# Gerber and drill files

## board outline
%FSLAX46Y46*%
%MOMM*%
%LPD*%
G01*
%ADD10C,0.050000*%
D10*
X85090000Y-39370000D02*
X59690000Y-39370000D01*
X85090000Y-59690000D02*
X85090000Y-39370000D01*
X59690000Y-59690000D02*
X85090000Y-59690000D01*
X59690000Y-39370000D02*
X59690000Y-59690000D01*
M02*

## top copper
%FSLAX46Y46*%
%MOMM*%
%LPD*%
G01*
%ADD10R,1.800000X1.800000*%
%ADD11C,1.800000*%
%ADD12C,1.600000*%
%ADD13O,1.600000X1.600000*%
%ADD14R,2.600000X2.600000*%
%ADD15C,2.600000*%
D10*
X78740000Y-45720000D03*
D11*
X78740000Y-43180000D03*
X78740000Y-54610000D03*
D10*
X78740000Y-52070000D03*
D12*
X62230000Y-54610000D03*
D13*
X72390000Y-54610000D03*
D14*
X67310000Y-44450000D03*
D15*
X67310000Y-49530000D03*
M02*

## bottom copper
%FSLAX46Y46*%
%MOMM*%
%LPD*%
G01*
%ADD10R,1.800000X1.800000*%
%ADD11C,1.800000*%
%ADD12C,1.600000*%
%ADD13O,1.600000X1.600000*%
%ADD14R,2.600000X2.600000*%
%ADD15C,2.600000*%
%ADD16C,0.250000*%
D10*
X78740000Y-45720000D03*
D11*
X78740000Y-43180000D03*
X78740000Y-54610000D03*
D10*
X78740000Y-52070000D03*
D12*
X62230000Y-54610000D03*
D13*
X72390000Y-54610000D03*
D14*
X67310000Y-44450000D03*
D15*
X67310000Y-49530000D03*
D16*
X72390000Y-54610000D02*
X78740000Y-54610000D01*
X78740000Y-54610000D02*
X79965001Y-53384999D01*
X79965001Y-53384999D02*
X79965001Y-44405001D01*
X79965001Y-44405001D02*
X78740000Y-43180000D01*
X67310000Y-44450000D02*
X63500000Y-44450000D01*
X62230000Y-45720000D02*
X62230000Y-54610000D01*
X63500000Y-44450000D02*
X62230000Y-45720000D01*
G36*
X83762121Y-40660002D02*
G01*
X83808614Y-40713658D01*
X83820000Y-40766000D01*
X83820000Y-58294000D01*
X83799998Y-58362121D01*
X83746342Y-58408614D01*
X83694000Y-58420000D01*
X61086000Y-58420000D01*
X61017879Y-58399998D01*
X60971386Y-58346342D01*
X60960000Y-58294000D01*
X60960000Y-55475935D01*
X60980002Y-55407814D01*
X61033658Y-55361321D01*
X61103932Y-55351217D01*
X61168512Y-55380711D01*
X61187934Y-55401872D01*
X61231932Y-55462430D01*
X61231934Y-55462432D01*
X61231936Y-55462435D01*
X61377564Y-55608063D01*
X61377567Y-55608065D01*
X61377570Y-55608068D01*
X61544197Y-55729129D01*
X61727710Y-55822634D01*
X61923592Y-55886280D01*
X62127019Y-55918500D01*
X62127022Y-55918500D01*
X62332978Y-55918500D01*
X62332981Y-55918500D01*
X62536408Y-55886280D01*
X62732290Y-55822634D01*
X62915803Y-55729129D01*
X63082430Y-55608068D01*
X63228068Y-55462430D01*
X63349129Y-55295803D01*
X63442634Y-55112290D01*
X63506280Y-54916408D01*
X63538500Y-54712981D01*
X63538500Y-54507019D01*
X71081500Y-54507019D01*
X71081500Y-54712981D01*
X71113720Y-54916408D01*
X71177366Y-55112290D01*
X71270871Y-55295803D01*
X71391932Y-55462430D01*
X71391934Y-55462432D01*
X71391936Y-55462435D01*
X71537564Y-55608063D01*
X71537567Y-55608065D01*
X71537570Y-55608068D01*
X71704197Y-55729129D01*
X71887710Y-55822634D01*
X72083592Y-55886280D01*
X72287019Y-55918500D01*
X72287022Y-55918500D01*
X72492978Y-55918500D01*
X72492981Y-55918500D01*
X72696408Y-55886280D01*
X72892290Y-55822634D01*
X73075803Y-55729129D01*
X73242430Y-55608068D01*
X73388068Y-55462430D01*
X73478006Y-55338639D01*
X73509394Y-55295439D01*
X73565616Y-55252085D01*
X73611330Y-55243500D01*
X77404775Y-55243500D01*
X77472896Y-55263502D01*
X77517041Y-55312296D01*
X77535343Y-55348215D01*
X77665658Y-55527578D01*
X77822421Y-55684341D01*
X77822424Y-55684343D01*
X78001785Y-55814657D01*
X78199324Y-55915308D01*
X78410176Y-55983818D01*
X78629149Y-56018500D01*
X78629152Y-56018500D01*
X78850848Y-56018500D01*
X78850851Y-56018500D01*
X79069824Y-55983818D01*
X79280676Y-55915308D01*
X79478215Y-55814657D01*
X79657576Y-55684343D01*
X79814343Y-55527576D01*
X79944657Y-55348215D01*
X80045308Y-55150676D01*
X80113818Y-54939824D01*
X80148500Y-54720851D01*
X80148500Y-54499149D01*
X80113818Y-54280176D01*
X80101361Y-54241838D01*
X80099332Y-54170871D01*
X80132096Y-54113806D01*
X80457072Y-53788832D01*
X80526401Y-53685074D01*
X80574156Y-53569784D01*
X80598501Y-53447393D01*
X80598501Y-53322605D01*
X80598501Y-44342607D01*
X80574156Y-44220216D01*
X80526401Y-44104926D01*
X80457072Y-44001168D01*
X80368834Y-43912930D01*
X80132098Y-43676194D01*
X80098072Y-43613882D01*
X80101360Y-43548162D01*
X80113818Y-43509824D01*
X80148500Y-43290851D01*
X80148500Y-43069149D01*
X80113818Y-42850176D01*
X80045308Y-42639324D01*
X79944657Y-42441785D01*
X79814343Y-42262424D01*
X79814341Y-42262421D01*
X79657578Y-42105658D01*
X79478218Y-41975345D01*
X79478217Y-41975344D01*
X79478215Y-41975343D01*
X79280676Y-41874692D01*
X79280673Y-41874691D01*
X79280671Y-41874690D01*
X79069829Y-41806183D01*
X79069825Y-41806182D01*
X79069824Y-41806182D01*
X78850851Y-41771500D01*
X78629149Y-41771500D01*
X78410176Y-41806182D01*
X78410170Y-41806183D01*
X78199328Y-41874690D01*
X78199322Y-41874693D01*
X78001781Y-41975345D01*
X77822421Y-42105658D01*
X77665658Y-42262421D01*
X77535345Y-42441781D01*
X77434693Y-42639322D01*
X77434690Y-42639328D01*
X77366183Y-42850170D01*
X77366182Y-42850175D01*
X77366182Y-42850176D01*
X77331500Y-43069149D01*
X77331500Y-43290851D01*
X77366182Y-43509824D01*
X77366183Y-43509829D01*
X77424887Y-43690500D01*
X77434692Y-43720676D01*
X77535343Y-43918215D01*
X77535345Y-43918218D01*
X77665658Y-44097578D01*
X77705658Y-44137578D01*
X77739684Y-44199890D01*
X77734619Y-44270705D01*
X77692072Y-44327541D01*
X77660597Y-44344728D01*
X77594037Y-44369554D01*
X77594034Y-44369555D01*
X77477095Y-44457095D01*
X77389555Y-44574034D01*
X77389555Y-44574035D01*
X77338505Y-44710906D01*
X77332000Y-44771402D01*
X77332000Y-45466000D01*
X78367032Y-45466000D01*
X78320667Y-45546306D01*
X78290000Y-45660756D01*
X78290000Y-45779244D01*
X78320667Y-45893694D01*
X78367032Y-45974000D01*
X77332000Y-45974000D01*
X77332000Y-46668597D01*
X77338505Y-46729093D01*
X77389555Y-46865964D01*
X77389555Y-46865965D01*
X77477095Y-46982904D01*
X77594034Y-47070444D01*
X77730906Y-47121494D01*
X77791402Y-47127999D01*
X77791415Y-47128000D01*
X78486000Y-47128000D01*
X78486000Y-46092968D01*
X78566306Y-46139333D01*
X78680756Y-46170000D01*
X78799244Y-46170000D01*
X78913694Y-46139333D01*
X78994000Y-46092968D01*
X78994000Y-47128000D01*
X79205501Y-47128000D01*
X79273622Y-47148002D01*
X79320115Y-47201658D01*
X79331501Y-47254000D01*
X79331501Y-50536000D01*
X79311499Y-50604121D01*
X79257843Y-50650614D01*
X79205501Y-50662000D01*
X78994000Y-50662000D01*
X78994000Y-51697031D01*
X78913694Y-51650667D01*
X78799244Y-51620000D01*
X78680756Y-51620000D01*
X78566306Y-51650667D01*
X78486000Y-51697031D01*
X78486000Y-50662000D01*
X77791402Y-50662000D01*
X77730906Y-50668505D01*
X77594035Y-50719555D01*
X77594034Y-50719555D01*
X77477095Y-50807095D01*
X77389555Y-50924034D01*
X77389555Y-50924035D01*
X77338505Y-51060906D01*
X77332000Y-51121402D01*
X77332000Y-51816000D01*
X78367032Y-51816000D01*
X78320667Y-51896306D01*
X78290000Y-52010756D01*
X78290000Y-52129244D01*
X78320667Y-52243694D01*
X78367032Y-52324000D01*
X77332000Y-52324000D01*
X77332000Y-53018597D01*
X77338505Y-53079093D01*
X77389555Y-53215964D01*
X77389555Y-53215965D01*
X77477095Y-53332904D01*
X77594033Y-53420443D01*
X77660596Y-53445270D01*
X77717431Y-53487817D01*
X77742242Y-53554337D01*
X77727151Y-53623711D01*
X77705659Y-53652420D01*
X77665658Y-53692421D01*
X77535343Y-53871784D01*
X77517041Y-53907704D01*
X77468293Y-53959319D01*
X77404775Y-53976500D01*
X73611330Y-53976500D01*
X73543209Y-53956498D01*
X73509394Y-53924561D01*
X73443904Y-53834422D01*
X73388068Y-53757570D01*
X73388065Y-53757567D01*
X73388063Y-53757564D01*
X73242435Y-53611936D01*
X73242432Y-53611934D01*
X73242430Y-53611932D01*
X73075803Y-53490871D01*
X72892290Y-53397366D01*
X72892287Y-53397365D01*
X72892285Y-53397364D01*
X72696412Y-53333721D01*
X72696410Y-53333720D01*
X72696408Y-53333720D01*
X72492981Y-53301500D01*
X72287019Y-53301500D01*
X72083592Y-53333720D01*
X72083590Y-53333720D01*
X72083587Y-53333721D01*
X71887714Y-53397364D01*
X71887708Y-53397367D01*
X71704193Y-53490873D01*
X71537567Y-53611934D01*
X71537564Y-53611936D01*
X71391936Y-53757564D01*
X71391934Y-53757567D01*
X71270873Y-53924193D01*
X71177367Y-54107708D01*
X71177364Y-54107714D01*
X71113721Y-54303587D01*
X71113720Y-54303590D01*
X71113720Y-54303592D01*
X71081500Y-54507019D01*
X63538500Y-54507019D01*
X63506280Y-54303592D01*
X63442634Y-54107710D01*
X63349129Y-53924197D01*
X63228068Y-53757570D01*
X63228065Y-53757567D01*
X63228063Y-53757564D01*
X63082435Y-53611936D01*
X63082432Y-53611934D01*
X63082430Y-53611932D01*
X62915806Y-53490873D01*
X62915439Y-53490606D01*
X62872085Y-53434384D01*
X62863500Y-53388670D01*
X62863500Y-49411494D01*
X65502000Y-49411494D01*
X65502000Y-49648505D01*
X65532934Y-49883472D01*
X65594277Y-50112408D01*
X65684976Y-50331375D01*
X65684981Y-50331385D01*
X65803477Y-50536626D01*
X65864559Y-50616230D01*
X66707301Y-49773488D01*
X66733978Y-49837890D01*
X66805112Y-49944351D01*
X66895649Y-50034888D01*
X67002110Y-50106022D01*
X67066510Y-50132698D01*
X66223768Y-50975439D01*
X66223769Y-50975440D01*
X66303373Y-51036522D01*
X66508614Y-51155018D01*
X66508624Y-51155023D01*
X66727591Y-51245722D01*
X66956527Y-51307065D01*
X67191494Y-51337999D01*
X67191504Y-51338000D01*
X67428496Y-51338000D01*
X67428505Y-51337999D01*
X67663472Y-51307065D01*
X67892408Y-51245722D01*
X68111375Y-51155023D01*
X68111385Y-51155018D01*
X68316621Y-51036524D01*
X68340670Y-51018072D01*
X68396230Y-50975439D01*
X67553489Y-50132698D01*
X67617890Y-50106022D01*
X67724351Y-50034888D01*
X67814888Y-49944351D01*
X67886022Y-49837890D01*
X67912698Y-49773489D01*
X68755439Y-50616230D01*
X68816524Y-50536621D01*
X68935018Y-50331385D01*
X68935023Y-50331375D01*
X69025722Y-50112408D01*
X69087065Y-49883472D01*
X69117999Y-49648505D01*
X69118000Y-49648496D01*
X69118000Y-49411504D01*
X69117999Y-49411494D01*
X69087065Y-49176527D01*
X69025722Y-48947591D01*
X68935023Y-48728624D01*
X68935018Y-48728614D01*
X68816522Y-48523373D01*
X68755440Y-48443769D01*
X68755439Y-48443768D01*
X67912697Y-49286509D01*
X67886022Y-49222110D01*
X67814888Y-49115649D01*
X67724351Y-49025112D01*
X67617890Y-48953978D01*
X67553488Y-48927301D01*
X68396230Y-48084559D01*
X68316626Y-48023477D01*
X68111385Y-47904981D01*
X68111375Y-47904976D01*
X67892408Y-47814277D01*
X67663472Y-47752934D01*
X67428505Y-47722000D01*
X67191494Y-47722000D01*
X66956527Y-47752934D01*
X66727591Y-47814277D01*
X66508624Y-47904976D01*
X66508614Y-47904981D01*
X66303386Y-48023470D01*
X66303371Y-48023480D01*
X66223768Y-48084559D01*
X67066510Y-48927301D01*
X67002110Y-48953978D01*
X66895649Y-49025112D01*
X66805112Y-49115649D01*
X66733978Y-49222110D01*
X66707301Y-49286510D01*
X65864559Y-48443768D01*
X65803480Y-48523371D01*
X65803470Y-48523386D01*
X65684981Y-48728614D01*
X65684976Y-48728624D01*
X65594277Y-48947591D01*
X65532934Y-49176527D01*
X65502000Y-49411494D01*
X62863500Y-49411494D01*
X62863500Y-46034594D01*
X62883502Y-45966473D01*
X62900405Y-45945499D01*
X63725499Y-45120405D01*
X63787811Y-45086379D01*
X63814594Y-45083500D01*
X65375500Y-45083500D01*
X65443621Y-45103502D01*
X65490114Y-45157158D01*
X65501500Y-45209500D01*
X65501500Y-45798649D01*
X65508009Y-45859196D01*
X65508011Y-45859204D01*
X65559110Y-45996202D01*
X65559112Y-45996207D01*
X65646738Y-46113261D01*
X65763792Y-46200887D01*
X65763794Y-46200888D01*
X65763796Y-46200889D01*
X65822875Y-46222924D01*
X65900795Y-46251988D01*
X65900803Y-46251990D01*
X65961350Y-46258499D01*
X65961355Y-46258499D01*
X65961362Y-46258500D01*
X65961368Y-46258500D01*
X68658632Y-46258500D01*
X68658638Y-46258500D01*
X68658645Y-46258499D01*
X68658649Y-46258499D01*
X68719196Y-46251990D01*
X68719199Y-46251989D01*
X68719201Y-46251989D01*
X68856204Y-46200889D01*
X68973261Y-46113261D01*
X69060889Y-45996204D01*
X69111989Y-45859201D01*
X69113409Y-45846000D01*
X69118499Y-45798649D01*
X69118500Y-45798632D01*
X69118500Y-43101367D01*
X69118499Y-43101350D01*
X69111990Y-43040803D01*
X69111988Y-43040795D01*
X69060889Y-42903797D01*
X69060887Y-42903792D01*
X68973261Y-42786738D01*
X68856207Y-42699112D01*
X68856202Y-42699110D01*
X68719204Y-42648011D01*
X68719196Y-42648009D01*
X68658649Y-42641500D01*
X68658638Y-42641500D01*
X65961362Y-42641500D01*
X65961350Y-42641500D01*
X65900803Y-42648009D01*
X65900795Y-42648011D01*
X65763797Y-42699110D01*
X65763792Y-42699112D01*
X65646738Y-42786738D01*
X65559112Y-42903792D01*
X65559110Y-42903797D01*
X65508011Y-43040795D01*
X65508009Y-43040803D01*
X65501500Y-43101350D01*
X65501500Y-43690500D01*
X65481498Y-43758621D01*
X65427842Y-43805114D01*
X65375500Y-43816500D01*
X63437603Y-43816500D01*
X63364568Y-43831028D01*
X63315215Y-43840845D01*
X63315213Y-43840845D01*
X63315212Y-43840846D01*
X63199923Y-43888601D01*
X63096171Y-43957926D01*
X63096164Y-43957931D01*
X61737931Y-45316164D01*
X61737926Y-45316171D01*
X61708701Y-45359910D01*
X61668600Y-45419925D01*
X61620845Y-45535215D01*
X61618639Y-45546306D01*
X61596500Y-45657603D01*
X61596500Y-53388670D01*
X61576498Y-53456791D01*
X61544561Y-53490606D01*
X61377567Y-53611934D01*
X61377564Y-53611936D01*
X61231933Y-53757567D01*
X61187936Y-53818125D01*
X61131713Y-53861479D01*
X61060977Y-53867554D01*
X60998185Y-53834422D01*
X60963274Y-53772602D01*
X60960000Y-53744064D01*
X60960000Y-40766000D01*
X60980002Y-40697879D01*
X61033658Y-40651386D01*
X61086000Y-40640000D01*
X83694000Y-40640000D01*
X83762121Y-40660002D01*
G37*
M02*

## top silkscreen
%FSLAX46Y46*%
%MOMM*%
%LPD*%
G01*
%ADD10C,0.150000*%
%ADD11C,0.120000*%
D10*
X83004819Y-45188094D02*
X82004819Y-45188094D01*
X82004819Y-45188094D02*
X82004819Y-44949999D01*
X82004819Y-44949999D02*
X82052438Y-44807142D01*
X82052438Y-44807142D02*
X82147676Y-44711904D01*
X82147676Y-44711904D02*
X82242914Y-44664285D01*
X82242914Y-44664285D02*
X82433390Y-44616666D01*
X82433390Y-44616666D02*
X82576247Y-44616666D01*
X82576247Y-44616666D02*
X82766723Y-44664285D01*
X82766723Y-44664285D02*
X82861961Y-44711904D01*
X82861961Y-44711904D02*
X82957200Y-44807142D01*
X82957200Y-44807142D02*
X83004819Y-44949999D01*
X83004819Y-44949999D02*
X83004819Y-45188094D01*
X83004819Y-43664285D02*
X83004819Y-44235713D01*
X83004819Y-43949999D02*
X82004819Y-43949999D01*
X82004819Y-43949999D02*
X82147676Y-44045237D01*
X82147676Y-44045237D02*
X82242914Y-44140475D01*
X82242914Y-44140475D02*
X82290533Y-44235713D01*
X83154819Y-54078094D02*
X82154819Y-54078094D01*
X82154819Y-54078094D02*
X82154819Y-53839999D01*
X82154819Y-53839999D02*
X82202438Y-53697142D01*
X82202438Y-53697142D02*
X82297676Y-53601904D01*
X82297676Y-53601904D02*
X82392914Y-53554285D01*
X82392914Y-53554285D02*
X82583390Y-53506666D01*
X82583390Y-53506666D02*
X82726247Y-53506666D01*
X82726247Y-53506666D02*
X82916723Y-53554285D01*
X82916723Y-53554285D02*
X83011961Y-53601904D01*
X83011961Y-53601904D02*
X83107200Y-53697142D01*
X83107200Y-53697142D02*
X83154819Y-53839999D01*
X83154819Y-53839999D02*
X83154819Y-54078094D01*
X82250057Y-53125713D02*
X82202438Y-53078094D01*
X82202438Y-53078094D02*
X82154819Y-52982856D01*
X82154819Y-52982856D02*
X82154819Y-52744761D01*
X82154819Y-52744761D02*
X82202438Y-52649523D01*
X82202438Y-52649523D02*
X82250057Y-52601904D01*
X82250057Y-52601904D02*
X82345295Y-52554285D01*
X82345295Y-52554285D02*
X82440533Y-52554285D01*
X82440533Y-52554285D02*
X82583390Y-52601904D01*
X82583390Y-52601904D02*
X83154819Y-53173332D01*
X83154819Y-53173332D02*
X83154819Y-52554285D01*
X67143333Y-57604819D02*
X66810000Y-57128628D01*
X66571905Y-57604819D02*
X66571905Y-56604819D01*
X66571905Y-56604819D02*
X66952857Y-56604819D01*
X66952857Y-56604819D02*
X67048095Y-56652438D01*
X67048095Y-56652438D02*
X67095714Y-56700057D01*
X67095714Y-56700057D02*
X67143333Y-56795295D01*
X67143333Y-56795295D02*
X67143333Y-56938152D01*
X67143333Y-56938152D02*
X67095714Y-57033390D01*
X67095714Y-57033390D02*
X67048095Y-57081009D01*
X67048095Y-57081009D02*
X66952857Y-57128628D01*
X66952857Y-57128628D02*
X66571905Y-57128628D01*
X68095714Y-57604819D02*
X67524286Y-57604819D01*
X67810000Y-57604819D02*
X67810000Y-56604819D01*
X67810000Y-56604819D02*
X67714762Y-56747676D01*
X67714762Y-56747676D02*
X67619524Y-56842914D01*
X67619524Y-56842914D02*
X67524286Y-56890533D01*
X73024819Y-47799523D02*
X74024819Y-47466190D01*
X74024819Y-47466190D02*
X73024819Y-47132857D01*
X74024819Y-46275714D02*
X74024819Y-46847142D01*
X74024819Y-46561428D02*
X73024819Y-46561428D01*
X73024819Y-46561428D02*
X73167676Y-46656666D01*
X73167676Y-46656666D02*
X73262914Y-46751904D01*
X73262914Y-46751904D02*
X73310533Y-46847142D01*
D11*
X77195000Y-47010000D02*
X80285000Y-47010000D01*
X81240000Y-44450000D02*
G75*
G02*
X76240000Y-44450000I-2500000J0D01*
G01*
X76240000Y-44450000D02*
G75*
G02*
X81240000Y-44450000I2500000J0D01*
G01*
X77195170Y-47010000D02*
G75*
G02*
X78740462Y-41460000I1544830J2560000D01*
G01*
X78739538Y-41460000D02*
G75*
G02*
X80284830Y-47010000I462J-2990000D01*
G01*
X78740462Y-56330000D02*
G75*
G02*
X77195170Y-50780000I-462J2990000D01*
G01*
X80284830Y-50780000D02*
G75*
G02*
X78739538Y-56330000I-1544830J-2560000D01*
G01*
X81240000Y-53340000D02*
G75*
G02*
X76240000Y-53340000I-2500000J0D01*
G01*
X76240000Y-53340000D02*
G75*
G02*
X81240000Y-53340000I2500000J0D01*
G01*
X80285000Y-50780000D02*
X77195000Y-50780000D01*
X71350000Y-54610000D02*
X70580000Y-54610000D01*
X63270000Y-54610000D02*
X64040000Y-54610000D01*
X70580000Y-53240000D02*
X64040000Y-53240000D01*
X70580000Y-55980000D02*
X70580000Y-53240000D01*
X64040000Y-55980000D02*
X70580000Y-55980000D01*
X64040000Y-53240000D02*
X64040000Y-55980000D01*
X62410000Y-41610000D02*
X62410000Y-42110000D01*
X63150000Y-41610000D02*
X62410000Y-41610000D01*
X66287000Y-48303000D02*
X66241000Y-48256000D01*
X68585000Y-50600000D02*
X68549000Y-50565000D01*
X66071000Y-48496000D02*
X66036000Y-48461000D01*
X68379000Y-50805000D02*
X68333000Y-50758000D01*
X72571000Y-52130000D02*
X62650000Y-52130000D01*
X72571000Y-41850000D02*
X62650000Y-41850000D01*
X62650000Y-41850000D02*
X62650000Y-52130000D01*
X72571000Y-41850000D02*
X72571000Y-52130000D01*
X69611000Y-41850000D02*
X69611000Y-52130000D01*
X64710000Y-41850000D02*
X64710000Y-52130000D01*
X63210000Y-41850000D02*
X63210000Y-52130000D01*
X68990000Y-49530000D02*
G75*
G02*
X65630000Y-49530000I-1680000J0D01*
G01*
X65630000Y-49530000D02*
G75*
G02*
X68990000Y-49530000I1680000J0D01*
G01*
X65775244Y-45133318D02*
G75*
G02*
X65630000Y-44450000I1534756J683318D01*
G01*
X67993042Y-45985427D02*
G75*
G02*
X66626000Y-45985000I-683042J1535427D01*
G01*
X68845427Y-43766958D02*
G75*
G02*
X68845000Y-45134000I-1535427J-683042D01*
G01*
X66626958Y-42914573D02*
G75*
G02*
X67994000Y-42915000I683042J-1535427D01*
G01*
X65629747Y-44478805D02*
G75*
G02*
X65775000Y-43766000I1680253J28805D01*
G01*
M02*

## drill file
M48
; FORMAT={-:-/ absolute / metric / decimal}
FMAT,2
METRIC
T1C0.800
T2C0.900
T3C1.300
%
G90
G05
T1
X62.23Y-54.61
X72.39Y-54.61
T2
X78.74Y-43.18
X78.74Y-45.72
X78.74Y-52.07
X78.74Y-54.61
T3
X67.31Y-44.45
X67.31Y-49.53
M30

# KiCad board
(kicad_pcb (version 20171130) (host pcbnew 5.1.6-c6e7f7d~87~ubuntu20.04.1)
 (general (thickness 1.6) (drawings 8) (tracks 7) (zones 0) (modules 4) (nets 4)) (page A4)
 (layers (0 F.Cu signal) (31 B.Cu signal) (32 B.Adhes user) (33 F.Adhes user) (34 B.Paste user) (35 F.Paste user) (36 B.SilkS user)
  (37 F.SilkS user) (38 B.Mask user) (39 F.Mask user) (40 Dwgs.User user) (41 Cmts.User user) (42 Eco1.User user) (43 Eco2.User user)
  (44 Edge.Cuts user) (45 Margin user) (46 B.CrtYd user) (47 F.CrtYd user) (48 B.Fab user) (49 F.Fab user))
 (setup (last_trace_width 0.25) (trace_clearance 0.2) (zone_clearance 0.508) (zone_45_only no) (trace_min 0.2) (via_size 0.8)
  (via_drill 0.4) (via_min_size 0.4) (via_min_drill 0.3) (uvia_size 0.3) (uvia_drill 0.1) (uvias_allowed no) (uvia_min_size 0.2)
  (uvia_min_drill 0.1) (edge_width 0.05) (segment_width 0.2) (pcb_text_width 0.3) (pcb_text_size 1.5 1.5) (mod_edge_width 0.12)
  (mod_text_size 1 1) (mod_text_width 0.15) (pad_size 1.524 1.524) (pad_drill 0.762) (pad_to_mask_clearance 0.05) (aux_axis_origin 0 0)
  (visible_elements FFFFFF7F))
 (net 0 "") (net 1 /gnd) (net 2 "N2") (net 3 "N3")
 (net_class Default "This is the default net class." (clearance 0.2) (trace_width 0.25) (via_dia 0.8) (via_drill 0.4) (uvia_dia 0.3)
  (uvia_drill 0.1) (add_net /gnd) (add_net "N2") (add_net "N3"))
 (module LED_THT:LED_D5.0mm (layer F.Cu) (at 78.74 45.72 90)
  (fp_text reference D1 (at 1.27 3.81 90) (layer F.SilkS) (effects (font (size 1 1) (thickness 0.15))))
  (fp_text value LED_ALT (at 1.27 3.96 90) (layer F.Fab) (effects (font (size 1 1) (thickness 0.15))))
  (fp_line (start -1.29 -1.545) (end -1.29 1.545) (layer F.SilkS) (width 0.12))
  (fp_circle (center 1.27 0) (end 3.77 0) (layer F.SilkS) (width 0.12))
  (fp_arc (start 1.27 0) (end -1.29 -1.54483) (angle 148.9) (layer F.SilkS) (width 0.12))
  (fp_arc (start 1.27 0) (end -1.29 1.54483) (angle -148.9) (layer F.SilkS) (width 0.12))
  (pad 1 thru_hole rect (at 0 0 90) (size 1.8 1.8) (drill 0.9) (layers *.Cu *.Mask) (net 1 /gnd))
  (pad 2 thru_hole circle (at 2.54 0 90) (size 1.8 1.8) (drill 0.9) (layers *.Cu *.Mask) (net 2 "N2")))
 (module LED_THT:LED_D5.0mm (layer F.Cu) (at 78.74 52.07 270)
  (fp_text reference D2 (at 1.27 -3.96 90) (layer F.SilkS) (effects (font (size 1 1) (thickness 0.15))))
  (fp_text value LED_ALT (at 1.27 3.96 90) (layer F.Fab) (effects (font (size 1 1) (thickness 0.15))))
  (fp_arc (start 1.27 0) (end -1.29 1.54483) (angle -148.9) (layer F.SilkS) (width 0.12))
  (fp_arc (start 1.27 0) (end -1.29 -1.54483) (angle 148.9) (layer F.SilkS) (width 0.12))
  (fp_circle (center 1.27 0) (end 3.77 0) (layer F.SilkS) (width 0.12))
  (fp_line (start -1.29 -1.545) (end -1.29 1.545) (layer F.SilkS) (width 0.12))
  (pad 2 thru_hole circle (at 2.54 0 270) (size 1.8 1.8) (drill 0.9) (layers *.Cu *.Mask) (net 2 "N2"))
  (pad 1 thru_hole rect (at 0 0 270) (size 1.8 1.8) (drill 0.9) (layers *.Cu *.Mask) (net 1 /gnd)))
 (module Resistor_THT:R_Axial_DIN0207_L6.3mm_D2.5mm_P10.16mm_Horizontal (layer F.Cu) (at 62.23 54.61)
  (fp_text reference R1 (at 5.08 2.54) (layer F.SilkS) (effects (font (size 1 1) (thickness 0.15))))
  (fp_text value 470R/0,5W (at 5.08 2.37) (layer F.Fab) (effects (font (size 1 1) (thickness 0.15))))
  (fp_line (start 9.12 0) (end 8.35 0) (layer F.SilkS) (width 0.12))
  (fp_line (start 1.04 0) (end 1.81 0) (layer F.SilkS) (width 0.12))
  (fp_line (start 8.35 -1.37) (end 1.81 -1.37) (layer F.SilkS) (width 0.12))
  (fp_line (start 8.35 1.37) (end 8.35 -1.37) (layer F.SilkS) (width 0.12))
  (fp_line (start 1.81 1.37) (end 8.35 1.37) (layer F.SilkS) (width 0.12))
  (fp_line (start 1.81 -1.37) (end 1.81 1.37) (layer F.SilkS) (width 0.12))
  (pad 1 thru_hole circle (at 0 0) (size 1.6 1.6) (drill 0.8) (layers *.Cu *.Mask) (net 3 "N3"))
  (pad 2 thru_hole oval (at 10.16 0) (size 1.6 1.6) (drill 0.8) (layers *.Cu *.Mask) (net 2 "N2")))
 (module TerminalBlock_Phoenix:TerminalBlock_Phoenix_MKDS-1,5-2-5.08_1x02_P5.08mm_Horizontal (layer F.Cu) (at 67.31 44.45 270)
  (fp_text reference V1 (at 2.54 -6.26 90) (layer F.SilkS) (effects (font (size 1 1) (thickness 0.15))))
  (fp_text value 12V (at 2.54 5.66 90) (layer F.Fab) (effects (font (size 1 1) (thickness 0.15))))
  (fp_line (start -2.84 4.9) (end -2.34 4.9) (layer F.SilkS) (width 0.12))
  (fp_line (start -2.84 4.16) (end -2.84 4.9) (layer F.SilkS) (width 0.12))
  (fp_line (start 3.853 1.023) (end 3.806 1.069) (layer F.SilkS) (width 0.12))
  (fp_line (start 6.15 -1.275) (end 6.115 -1.239) (layer F.SilkS) (width 0.12))
  (fp_line (start 4.046 1.239) (end 4.011 1.274) (layer F.SilkS) (width 0.12))
  (fp_line (start 6.355 -1.069) (end 6.308 -1.023) (layer F.SilkS) (width 0.12))
  (fp_line (start 7.68 -5.261) (end 7.68 4.66) (layer F.SilkS) (width 0.12))
  (fp_line (start -2.6 -5.261) (end -2.6 4.66) (layer F.SilkS) (width 0.12))
  (fp_line (start -2.6 4.66) (end 7.68 4.66) (layer F.SilkS) (width 0.12))
  (fp_line (start -2.6 -5.261) (end 7.68 -5.261) (layer F.SilkS) (width 0.12))
  (fp_line (start -2.6 -2.301) (end 7.68 -2.301) (layer F.SilkS) (width 0.12))
  (fp_line (start -2.6 2.6) (end 7.68 2.6) (layer F.SilkS) (width 0.12))
  (fp_line (start -2.6 4.1) (end 7.68 4.1) (layer F.SilkS) (width 0.12))
  (fp_circle (center 5.08 0) (end 6.76 0) (layer F.SilkS) (width 0.12))
  (fp_arc (start 0 0) (end 0 1.68) (angle -24) (layer F.SilkS) (width 0.12))
  (fp_arc (start 0 0) (end 1.535 0.684) (angle -48) (layer F.SilkS) (width 0.12))
  (fp_arc (start 0 0) (end 0.684 -1.535) (angle -48) (layer F.SilkS) (width 0.12))
  (fp_arc (start 0 0) (end -1.535 -0.684) (angle -48) (layer F.SilkS) (width 0.12))
  (fp_arc (start 0 0) (end -0.684 1.535) (angle -25) (layer F.SilkS) (width 0.12))
  (pad 1 thru_hole rect (at 0 0 270) (size 2.6 2.6) (drill 1.3) (layers *.Cu *.Mask) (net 3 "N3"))
  (pad 2 thru_hole circle (at 5.08 0 270) (size 2.6 2.6) (drill 1.3) (layers *.Cu *.Mask) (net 1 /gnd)))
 (gr_line (start 85.09 39.37) (end 59.69 39.37) (layer Edge.Cuts) (width 0.05))
 (gr_line (start 85.09 59.69) (end 85.09 39.37) (layer Edge.Cuts) (width 0.05))
 (gr_line (start 59.69 59.69) (end 85.09 59.69) (layer Edge.Cuts) (width 0.05))
 (gr_line (start 59.69 39.37) (end 59.69 59.69) (layer Edge.Cuts) (width 0.05))
 (segment (start 72.39 54.61) (end 78.74 54.61) (width 0.25) (layer B.Cu) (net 2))
 (segment (start 78.74 54.61) (end 79.965001 53.384999) (width 0.25) (layer B.Cu) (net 2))
 (segment (start 79.965001 53.384999) (end 79.965001 44.405001) (width 0.25) (layer B.Cu) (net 2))
 (segment (start 79.965001 44.405001) (end 78.74 43.18) (width 0.25) (layer B.Cu) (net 2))
 (segment (start 67.31 44.45) (end 63.5 44.45) (width 0.25) (layer B.Cu) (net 3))
 (segment (start 62.23 45.72) (end 62.23 54.61) (width 0.25) (layer B.Cu) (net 3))
 (segment (start 63.5 44.45) (end 62.23 45.72) (width 0.25) (layer B.Cu) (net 3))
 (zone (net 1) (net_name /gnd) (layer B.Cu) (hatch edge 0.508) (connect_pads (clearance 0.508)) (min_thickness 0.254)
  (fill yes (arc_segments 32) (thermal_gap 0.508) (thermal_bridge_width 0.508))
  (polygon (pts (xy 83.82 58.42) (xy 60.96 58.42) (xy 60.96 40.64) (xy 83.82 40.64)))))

